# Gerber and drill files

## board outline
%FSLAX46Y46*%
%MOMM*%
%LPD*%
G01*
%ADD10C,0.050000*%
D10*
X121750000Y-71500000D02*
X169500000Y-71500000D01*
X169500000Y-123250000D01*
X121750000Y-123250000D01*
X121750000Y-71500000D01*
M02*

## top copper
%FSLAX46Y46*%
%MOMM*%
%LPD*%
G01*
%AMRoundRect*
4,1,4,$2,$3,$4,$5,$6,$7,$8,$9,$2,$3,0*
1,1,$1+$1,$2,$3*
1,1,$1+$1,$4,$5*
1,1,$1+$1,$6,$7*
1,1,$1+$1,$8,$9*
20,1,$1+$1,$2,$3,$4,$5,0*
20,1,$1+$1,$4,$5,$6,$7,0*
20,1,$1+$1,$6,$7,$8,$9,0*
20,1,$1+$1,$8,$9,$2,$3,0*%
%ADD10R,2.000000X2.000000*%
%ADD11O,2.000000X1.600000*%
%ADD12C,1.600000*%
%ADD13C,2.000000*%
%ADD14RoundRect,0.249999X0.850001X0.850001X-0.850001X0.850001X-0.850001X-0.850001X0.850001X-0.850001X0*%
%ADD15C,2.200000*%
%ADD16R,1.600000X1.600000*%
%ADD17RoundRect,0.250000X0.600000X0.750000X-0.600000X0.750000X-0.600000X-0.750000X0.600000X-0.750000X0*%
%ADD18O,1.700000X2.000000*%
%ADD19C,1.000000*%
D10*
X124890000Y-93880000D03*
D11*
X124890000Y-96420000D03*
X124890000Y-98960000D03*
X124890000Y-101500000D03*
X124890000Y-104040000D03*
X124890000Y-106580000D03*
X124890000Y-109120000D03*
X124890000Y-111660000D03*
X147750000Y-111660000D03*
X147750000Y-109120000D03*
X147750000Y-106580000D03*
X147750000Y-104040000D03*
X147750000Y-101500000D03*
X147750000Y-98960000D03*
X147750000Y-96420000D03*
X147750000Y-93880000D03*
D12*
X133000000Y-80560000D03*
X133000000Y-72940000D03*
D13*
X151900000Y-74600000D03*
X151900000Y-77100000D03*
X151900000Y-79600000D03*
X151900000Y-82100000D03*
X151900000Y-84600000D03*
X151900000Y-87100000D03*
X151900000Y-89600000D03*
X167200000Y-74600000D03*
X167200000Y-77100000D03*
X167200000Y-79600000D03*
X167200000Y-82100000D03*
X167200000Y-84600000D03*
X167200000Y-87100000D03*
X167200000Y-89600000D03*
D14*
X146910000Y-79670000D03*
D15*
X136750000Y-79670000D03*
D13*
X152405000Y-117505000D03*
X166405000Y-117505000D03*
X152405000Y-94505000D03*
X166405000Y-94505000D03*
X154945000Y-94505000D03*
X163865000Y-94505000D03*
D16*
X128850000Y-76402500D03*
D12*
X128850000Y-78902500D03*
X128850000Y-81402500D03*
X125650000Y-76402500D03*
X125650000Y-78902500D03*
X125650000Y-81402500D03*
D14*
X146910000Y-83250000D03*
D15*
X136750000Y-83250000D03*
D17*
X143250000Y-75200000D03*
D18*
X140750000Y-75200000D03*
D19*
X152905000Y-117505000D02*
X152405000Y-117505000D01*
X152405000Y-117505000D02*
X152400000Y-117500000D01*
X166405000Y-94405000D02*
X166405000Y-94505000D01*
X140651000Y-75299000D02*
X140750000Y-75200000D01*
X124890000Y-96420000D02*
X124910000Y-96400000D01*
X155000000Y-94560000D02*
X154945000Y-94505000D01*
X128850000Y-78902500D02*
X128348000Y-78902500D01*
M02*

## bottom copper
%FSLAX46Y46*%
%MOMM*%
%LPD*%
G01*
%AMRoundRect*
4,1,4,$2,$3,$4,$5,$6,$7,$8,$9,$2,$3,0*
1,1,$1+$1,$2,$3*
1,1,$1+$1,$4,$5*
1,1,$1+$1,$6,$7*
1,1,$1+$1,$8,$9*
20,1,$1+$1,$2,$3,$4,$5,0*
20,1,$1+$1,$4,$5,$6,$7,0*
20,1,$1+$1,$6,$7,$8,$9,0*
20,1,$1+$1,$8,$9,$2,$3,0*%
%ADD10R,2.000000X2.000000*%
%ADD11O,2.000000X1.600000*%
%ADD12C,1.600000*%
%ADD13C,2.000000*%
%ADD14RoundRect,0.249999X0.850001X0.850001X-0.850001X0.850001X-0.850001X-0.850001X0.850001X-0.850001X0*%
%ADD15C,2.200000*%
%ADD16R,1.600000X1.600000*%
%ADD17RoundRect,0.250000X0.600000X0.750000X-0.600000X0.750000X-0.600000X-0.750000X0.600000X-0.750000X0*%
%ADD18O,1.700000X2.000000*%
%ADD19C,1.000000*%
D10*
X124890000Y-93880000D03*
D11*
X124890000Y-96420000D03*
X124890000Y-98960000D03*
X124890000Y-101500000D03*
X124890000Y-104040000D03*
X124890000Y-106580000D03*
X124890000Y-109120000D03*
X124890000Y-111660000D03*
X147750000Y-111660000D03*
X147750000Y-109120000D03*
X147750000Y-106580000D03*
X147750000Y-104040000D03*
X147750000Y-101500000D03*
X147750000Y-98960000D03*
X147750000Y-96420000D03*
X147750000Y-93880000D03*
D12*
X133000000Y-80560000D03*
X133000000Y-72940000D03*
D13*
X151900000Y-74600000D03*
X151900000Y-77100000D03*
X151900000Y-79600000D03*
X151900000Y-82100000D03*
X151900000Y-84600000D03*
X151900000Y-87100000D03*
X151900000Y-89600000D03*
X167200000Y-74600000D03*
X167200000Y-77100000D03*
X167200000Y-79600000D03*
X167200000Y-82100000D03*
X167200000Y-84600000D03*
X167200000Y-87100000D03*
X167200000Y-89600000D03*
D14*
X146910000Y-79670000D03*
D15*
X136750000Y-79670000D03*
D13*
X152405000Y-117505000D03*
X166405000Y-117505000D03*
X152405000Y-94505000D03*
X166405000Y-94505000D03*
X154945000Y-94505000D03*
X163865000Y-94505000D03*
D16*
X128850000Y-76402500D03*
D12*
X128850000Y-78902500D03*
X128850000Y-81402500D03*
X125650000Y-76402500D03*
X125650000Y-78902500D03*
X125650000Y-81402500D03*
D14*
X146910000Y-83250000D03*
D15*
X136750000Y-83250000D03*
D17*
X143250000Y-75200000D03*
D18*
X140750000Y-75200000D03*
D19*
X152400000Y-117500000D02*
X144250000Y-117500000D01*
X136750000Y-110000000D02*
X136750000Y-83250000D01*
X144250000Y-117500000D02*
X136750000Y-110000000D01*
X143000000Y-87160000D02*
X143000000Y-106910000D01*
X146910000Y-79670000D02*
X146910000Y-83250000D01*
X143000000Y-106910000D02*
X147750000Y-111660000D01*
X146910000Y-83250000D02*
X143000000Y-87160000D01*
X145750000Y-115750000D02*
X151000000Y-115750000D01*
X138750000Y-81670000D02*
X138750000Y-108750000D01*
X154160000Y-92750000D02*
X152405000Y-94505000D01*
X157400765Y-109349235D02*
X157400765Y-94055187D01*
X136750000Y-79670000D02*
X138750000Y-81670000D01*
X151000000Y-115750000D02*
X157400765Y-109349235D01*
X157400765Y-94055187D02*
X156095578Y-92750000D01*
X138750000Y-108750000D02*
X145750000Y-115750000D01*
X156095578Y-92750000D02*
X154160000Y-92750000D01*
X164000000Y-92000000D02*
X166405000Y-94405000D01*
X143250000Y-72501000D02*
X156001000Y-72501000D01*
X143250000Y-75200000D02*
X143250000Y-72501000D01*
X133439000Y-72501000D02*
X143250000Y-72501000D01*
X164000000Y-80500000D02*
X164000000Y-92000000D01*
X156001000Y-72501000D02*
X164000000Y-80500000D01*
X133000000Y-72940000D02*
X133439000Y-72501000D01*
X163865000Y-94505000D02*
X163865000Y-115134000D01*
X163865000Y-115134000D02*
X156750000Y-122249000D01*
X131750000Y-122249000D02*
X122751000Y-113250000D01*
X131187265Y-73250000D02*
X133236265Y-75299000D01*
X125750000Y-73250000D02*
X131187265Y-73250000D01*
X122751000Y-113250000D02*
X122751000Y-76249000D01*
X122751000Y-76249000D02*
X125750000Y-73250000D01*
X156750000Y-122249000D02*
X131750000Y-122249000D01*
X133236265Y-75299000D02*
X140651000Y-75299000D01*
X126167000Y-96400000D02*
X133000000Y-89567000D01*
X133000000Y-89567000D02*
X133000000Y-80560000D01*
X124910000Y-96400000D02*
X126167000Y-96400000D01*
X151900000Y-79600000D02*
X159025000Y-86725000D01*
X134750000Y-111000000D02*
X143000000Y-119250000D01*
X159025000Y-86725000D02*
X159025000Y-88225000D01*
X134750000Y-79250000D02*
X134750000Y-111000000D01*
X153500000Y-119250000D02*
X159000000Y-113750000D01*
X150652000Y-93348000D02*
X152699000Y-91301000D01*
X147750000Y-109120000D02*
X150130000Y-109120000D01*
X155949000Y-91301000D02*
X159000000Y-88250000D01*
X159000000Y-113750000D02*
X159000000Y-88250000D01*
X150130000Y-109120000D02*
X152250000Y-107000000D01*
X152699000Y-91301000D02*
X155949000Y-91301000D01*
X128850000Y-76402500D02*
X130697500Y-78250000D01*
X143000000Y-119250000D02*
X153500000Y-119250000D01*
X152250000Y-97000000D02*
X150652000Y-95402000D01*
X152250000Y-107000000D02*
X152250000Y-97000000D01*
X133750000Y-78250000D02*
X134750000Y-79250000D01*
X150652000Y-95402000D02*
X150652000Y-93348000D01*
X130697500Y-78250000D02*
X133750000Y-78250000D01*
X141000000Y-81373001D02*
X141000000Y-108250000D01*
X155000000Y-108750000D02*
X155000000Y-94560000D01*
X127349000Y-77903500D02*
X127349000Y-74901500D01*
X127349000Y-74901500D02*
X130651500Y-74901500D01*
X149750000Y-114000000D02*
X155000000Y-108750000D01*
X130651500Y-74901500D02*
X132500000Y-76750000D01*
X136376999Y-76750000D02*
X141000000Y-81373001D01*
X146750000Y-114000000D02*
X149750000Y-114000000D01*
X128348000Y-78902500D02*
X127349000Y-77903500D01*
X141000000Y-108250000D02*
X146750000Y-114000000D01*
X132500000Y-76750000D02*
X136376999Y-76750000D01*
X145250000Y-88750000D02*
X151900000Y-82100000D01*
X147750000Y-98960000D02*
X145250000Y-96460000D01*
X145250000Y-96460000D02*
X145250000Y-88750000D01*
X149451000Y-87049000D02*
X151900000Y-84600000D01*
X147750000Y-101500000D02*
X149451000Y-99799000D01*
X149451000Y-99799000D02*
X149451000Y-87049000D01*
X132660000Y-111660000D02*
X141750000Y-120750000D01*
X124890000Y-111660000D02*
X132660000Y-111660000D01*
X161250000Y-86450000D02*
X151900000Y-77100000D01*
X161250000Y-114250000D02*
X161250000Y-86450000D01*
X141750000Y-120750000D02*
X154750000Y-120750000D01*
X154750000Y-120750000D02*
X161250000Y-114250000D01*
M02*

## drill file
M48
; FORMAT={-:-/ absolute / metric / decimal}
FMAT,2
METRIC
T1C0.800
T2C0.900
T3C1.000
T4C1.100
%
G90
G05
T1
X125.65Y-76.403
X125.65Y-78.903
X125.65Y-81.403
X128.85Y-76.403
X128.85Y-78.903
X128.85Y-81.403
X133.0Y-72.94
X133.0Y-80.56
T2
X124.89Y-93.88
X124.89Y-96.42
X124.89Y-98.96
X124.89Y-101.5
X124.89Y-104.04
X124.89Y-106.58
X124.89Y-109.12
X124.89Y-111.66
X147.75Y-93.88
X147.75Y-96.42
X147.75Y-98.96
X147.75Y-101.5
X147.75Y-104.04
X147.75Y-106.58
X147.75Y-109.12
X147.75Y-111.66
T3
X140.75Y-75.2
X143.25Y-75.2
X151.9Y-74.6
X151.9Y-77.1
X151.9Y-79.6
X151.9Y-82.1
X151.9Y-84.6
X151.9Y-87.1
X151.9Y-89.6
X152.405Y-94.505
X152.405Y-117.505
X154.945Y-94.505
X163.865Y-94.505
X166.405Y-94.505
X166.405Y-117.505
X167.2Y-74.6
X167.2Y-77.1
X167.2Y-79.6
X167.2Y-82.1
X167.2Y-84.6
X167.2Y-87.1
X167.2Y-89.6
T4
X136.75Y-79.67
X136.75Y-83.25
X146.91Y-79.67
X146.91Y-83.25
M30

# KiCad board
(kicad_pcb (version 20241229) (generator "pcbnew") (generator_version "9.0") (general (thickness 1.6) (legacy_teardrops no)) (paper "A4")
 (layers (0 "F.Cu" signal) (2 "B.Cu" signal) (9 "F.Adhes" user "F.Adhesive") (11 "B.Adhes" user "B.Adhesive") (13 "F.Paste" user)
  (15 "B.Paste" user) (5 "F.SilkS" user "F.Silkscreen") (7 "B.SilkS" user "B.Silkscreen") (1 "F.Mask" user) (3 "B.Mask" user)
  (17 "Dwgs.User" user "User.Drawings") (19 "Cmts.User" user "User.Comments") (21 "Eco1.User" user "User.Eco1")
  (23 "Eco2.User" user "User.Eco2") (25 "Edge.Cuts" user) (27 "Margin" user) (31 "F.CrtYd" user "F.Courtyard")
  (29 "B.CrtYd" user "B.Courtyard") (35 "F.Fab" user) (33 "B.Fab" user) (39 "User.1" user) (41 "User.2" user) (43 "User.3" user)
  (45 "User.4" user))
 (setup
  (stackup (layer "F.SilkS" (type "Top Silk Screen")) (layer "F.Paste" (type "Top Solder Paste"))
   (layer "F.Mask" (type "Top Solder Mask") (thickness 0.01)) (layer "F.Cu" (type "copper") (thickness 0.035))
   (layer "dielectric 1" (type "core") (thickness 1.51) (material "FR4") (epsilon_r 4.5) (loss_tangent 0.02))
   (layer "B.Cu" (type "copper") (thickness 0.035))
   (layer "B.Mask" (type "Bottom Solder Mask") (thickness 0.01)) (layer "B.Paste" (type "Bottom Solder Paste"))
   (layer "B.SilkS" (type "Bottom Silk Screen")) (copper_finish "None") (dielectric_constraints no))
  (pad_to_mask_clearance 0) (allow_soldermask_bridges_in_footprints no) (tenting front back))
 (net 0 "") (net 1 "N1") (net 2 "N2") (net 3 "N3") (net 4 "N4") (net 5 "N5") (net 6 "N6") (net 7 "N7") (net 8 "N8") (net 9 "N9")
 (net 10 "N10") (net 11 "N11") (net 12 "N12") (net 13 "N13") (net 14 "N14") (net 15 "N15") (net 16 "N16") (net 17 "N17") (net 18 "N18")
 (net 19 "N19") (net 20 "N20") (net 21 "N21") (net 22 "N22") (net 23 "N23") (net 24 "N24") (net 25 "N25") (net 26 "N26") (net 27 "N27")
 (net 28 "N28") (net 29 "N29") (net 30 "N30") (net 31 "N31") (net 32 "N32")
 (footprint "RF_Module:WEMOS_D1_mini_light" (layer "F.Cu") (at 124.89 93.88)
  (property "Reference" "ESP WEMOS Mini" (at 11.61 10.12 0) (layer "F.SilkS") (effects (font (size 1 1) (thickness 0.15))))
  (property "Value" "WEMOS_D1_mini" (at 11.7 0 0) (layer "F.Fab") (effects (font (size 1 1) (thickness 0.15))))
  (pad "1" thru_hole rect (at 0 0) (size 2 2) (drill 0.9) (layers "*.Cu" "*.Mask") (remove_unused_layers no) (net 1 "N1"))
  (pad "2" thru_hole oval (at 0 2.54) (size 2 1.6) (drill 0.9) (layers "*.Cu" "*.Mask") (remove_unused_layers no) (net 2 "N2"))
  (pad "3" thru_hole oval (at 0 5.08) (size 2 1.6) (drill 0.9) (layers "*.Cu" "*.Mask") (remove_unused_layers no) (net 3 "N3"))
  (pad "4" thru_hole oval (at 0 7.62) (size 2 1.6) (drill 0.9) (layers "*.Cu" "*.Mask") (remove_unused_layers no) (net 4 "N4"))
  (pad "5" thru_hole oval (at 0 10.16) (size 2 1.6) (drill 0.9) (layers "*.Cu" "*.Mask") (remove_unused_layers no) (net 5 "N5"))
  (pad "6" thru_hole oval (at 0 12.7) (size 2 1.6) (drill 0.9) (layers "*.Cu" "*.Mask") (remove_unused_layers no) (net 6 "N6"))
  (pad "7" thru_hole oval (at 0 15.24) (size 2 1.6) (drill 0.9) (layers "*.Cu" "*.Mask") (remove_unused_layers no) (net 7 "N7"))
  (pad "8" thru_hole oval (at 0 17.78) (size 2 1.6) (drill 0.9) (layers "*.Cu" "*.Mask") (remove_unused_layers no) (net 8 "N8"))
  (pad "9" thru_hole oval (at 22.86 17.78) (size 2 1.6) (drill 0.9) (layers "*.Cu" "*.Mask") (remove_unused_layers no) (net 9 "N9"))
  (pad "10" thru_hole oval (at 22.86 15.24) (size 2 1.6) (drill 0.9) (layers "*.Cu" "*.Mask") (remove_unused_layers no) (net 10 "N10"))
  (pad "11" thru_hole oval (at 22.86 12.7) (size 2 1.6) (drill 0.9) (layers "*.Cu" "*.Mask") (remove_unused_layers no) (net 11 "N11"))
  (pad "12" thru_hole oval (at 22.86 10.16) (size 2 1.6) (drill 0.9) (layers "*.Cu" "*.Mask") (remove_unused_layers no) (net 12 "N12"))
  (pad "13" thru_hole oval (at 22.86 7.62) (size 2 1.6) (drill 0.9) (layers "*.Cu" "*.Mask") (remove_unused_layers no) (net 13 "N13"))
  (pad "14" thru_hole oval (at 22.86 5.08) (size 2 1.6) (drill 0.9) (layers "*.Cu" "*.Mask") (remove_unused_layers no) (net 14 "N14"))
  (pad "15" thru_hole oval (at 22.86 2.54) (size 2 1.6) (drill 0.9) (layers "*.Cu" "*.Mask") (remove_unused_layers no) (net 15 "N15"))
  (pad "16" thru_hole oval (at 22.86 0) (size 2 1.6) (drill 0.9) (layers "*.Cu" "*.Mask") (remove_unused_layers no) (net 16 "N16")))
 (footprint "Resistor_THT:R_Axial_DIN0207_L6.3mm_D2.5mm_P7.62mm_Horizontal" (layer "F.Cu") (at 133 80.56 90)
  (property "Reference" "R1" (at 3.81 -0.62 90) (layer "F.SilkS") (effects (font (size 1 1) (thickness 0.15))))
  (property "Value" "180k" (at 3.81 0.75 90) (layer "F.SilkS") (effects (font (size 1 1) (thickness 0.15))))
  (pad "1" thru_hole circle (at 0 0 90) (size 1.6 1.6) (drill 0.8) (layers "*.Cu" "*.Mask") (remove_unused_layers no) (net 2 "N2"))
  (pad "2" thru_hole circle (at 7.62 0 90) (size 1.6 1.6) (drill 0.8) (layers "*.Cu" "*.Mask") (remove_unused_layers no) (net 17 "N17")))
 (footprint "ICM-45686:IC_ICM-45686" (layer "F.Cu") (at 160.5 82)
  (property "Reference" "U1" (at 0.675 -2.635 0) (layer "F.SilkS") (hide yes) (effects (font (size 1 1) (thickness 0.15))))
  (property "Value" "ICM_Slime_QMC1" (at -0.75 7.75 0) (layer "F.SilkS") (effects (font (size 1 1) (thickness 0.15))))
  (pad "1" thru_hole circle (at -8.6 -7.4) (size 2 2) (drill 1) (layers "*.Cu" "*.Mask") (remove_unused_layers no) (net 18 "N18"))
  (pad "2" thru_hole circle (at -8.6 -4.9) (size 2 2) (drill 1) (layers "*.Cu" "*.Mask") (remove_unused_layers no) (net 8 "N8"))
  (pad "3" thru_hole circle (at -8.6 -2.4) (size 2 2) (drill 1) (layers "*.Cu" "*.Mask") (remove_unused_layers no) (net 10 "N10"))
  (pad "4" thru_hole circle (at -8.6 0.1) (size 2 2) (drill 1) (layers "*.Cu" "*.Mask") (remove_unused_layers no) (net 14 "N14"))
  (pad "5" thru_hole circle (at -8.6 2.6) (size 2 2) (drill 1) (layers "*.Cu" "*.Mask") (remove_unused_layers no) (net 13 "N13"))
  (pad "6" thru_hole circle (at -8.6 5.1) (size 2 2) (drill 1) (layers "*.Cu" "*.Mask") (remove_unused_layers no) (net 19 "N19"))
  (pad "7" thru_hole circle (at -8.6 7.6) (size 2 2) (drill 1) (layers "*.Cu" "*.Mask") (remove_unused_layers no) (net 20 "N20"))
  (pad "8" thru_hole circle (at 6.7 -7.4) (size 2 2) (drill 1) (layers "*.Cu" "*.Mask") (remove_unused_layers no) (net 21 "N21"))
  (pad "9" thru_hole circle (at 6.7 -4.9) (size 2 2) (drill 1) (layers "*.Cu" "*.Mask") (remove_unused_layers no) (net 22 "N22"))
  (pad "10" thru_hole circle (at 6.7 -2.4) (size 2 2) (drill 1) (layers "*.Cu" "*.Mask") (remove_unused_layers no) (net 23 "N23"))
  (pad "11" thru_hole circle (at 6.7 0.1) (size 2 2) (drill 1) (layers "*.Cu" "*.Mask") (remove_unused_layers no) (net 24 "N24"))
  (pad "12" thru_hole circle (at 6.7 2.6) (size 2 2) (drill 1) (layers "*.Cu" "*.Mask") (remove_unused_layers no) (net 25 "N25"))
  (pad "13" thru_hole circle (at 6.7 5.1) (size 2 2) (drill 1) (layers "*.Cu" "*.Mask") (remove_unused_layers no) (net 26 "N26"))
  (pad "14" thru_hole circle (at 6.7 7.6) (size 2 2) (drill 1) (layers "*.Cu" "*.Mask") (remove_unused_layers no) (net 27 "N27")))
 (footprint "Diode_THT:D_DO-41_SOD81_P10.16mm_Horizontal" (layer "F.Cu") (at 146.91 79.67 180)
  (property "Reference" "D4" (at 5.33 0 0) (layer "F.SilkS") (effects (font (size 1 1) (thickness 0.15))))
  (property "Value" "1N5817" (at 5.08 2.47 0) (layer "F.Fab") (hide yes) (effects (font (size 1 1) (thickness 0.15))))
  (pad "1" thru_hole roundrect (at 0 0 180) (size 2.2 2.2) (drill 1.1) (layers "*.Cu" "*.Mask") (remove_unused_layers no)
   (roundrect_rratio 0.113636) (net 9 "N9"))
  (pad "2" thru_hole circle (at 10.16 0 180) (size 2.2 2.2) (drill 1.1) (layers "*.Cu" "*.Mask") (remove_unused_layers no) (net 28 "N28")))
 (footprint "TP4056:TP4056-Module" (layer "F.Cu") (at 168.005 120.005 90)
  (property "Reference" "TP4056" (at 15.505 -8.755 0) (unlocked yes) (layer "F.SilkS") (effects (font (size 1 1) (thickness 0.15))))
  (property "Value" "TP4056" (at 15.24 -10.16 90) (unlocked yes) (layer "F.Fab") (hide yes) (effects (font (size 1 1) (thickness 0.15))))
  (pad "1" thru_hole circle (at 2.5 -15.6 90) (size 2 2) (drill 1) (layers "*.Cu" "*.Mask") (remove_unused_layers no) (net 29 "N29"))
  (pad "2" thru_hole circle (at 2.5 -1.6 90) (size 2 2) (drill 1) (layers "*.Cu" "*.Mask") (remove_unused_layers no) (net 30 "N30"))
  (pad "3" thru_hole circle (at 25.5 -15.6 90) (size 2 2) (drill 1) (layers "*.Cu" "*.Mask") (remove_unused_layers no) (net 28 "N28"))
  (pad "4" thru_hole circle (at 25.5 -1.6 90) (size 2 2) (drill 1) (layers "*.Cu" "*.Mask") (remove_unused_layers no) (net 17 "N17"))
  (pad "5" thru_hole circle (at 25.5 -13.06 90) (size 2 2) (drill 1) (layers "*.Cu" "*.Mask") (remove_unused_layers no) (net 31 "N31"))
  (pad "6" thru_hole circle (at 25.5 -4.14 90) (size 2 2) (drill 1) (layers "*.Cu" "*.Mask") (remove_unused_layers no) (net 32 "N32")))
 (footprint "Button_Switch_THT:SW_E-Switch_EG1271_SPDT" (layer "F.Cu") (at 128.85 76.4025 -90)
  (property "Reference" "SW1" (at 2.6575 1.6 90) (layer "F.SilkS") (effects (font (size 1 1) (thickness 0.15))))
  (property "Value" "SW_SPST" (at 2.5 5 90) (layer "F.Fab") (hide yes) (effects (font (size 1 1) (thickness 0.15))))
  (pad "1" thru_hole rect (at 0 0 270) (size 1.6 1.6) (drill 0.8) (layers "*.Cu" "*.Mask") (remove_unused_layers no) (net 10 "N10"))
  (pad "2" thru_hole circle (at 2.5 0 270) (size 1.6 1.6) (drill 0.8) (layers "*.Cu" "*.Mask") (remove_unused_layers no) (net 31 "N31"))
  (pad "3" thru_hole circle (at 5 0 270) (size 1.6 1.6) (drill 0.8) (layers "*.Cu" "*.Mask") (remove_unused_layers no))
  (pad "4" thru_hole circle (at 0 3.2 270) (size 1.6 1.6) (drill 0.8) (layers "*.Cu" "*.Mask") (remove_unused_layers no))
  (pad "5" thru_hole circle (at 2.5 3.2 270) (size 1.6 1.6) (drill 0.8) (layers "*.Cu" "*.Mask") (remove_unused_layers no))
  (pad "6" thru_hole circle (at 5 3.2 270) (size 1.6 1.6) (drill 0.8) (layers "*.Cu" "*.Mask") (remove_unused_layers no)))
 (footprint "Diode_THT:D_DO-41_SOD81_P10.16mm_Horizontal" (layer "F.Cu") (at 146.91 83.25 180)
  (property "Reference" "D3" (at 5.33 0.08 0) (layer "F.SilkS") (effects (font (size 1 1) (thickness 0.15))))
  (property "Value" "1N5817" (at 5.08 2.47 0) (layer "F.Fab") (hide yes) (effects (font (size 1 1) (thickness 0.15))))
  (pad "1" thru_hole roundrect (at 0 0 180) (size 2.2 2.2) (drill 1.1) (layers "*.Cu" "*.Mask") (remove_unused_layers no)
   (roundrect_rratio 0.113636) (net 9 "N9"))
  (pad "2" thru_hole circle (at 10.16 0 180) (size 2.2 2.2) (drill 1.1) (layers "*.Cu" "*.Mask") (remove_unused_layers no) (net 29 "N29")))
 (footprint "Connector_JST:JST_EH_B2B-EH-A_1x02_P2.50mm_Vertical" (layer "B.Cu") (at 143.25 75.2 180)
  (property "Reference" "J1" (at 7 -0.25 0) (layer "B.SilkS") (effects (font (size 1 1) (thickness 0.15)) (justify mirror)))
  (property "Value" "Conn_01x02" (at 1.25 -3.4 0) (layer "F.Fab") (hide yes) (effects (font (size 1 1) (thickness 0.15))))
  (pad "1" thru_hole roundrect (at 0 0 180) (size 1.7 2) (drill 1) (layers "*.Cu" "*.Mask") (remove_unused_layers no)
   (roundrect_rratio 0.147059) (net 17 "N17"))
  (pad "2" thru_hole oval (at 2.5 0 180) (size 1.7 2) (drill 1) (layers "*.Cu" "*.Mask") (remove_unused_layers no) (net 32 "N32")))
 (gr_rect (start 121.75 71.5) (end 169.5 123.25) (stroke (width 0.05) (type default)) (fill no) (locked yes) (layer "Edge.Cuts"))
 (segment (start 152.905 117.505) (end 152.405 117.505) (width 1) (layer "F.Cu") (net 29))
 (segment (start 152.405 117.505) (end 152.4 117.5) (width 1) (layer "F.Cu") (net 29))
 (segment (start 152.4 117.5) (end 144.25 117.5) (width 1) (layer "B.Cu") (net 29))
 (segment (start 136.75 110) (end 136.75 83.25) (width 1) (layer "B.Cu") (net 29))
 (segment (start 144.25 117.5) (end 136.75 110) (width 1) (layer "B.Cu") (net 29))
 (segment (start 143 87.16) (end 143 106.91) (width 1) (layer "B.Cu") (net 9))
 (segment (start 146.91 79.67) (end 146.91 83.25) (width 1) (layer "B.Cu") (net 9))
 (segment (start 143 106.91) (end 147.75 111.66) (width 1) (layer "B.Cu") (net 9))
 (segment (start 146.91 83.25) (end 143 87.16) (width 1) (layer "B.Cu") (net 9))
 (segment (start 145.75 115.75) (end 151 115.75) (width 1) (layer "B.Cu") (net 28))
 (segment (start 138.75 81.67) (end 138.75 108.75) (width 1) (layer "B.Cu") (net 28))
 (segment (start 154.16 92.75) (end 152.405 94.505) (width 1) (layer "B.Cu") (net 28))
 (segment (start 157.400765 109.349235) (end 157.400765 94.055187) (width 1) (layer "B.Cu") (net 28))
 (segment (start 136.75 79.67) (end 138.75 81.67) (width 1) (layer "B.Cu") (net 28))
 (segment (start 151 115.75) (end 157.400765 109.349235) (width 1) (layer "B.Cu") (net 28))
 (segment (start 157.400765 94.055187) (end 156.095578 92.75) (width 1) (layer "B.Cu") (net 28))
 (segment (start 138.75 108.75) (end 145.75 115.75) (width 1) (layer "B.Cu") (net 28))
 (segment (start 156.095578 92.75) (end 154.16 92.75) (width 1) (layer "B.Cu") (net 28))
 (segment (start 166.405 94.405) (end 166.405 94.505) (width 1) (layer "F.Cu") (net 17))
 (segment (start 164 92) (end 166.405 94.405) (width 1) (layer "B.Cu") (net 17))
 (segment (start 143.25 72.501) (end 156.001 72.501) (width 1) (layer "B.Cu") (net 17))
 (segment (start 143.25 75.2) (end 143.25 72.501) (width 1) (layer "B.Cu") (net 17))
 (segment (start 133.439 72.501) (end 143.25 72.501) (width 1) (layer "B.Cu") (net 17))
 (segment (start 164 80.5) (end 164 92) (width 1) (layer "B.Cu") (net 17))
 (segment (start 156.001 72.501) (end 164 80.5) (width 1) (layer "B.Cu") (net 17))
 (segment (start 133 72.94) (end 133.439 72.501) (width 1) (layer "B.Cu") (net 17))
 (segment (start 140.651 75.299) (end 140.75 75.2) (width 1) (layer "F.Cu") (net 32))
 (segment (start 163.865 94.505) (end 163.865 115.134) (width 1) (layer "B.Cu") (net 32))
 (segment (start 163.865 115.134) (end 156.75 122.249) (width 1) (layer "B.Cu") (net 32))
 (segment (start 131.75 122.249) (end 122.751 113.25) (width 1) (layer "B.Cu") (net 32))
 (segment (start 131.187265 73.25) (end 133.236265 75.299) (width 1) (layer "B.Cu") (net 32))
 (segment (start 125.75 73.25) (end 131.187265 73.25) (width 1) (layer "B.Cu") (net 32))
 (segment (start 122.751 113.25) (end 122.751 76.249) (width 1) (layer "B.Cu") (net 32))
 (segment (start 122.751 76.249) (end 125.75 73.25) (width 1) (layer "B.Cu") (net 32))
 (segment (start 156.75 122.249) (end 131.75 122.249) (width 1) (layer "B.Cu") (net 32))
 (segment (start 133.236265 75.299) (end 140.651 75.299) (width 1) (layer "B.Cu") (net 32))
 (segment (start 124.89 96.42) (end 124.91 96.4) (width 1) (layer "F.Cu") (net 2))
 (segment (start 126.167 96.4) (end 133 89.567) (width 1) (layer "B.Cu") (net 2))
 (segment (start 133 89.567) (end 133 80.56) (width 1) (layer "B.Cu") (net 2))
 (segment (start 124.91 96.4) (end 126.167 96.4) (width 1) (layer "B.Cu") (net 2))
 (segment (start 151.9 79.6) (end 159.025 86.725) (width 1) (layer "B.Cu") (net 10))
 (segment (start 134.75 111) (end 143 119.25) (width 1) (layer "B.Cu") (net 10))
 (segment (start 159.025 86.725) (end 159.025 88.225) (width 1) (layer "B.Cu") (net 10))
 (segment (start 134.75 79.25) (end 134.75 111) (width 1) (layer "B.Cu") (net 10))
 (segment (start 153.5 119.25) (end 159 113.75) (width 1) (layer "B.Cu") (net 10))
 (segment (start 150.652 93.348) (end 152.699 91.301) (width 1) (layer "B.Cu") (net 10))
 (segment (start 147.75 109.12) (end 150.13 109.12) (width 1) (layer "B.Cu") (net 10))
 (segment (start 155.949 91.301) (end 159 88.25) (width 1) (layer "B.Cu") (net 10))
 (segment (start 159 113.75) (end 159 88.25) (width 1) (layer "B.Cu") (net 10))
 (segment (start 150.13 109.12) (end 152.25 107) (width 1) (layer "B.Cu") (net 10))
 (segment (start 152.699 91.301) (end 155.949 91.301) (width 1) (layer "B.Cu") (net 10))
 (segment (start 128.85 76.4025) (end 130.6975 78.25) (width 1) (layer "B.Cu") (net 10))
 (segment (start 143 119.25) (end 153.5 119.25) (width 1) (layer "B.Cu") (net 10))
 (segment (start 152.25 97) (end 150.652 95.402) (width 1) (layer "B.Cu") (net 10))
 (segment (start 152.25 107) (end 152.25 97) (width 1) (layer "B.Cu") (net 10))
 (segment (start 133.75 78.25) (end 134.75 79.25) (width 1) (layer "B.Cu") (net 10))
 (segment (start 150.652 95.402) (end 150.652 93.348) (width 1) (layer "B.Cu") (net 10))
 (segment (start 130.6975 78.25) (end 133.75 78.25) (width 1) (layer "B.Cu") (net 10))
 (segment (start 155 94.56) (end 154.945 94.505) (width 1) (layer "F.Cu") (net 31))
 (segment (start 128.85 78.9025) (end 128.348 78.9025) (width 1) (layer "F.Cu") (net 31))
 (segment (start 141 81.373001) (end 141 108.25) (width 1) (layer "B.Cu") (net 31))
 (segment (start 155 108.75) (end 155 94.56) (width 1) (layer "B.Cu") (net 31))
 (segment (start 127.349 77.9035) (end 127.349 74.9015) (width 1) (layer "B.Cu") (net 31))
 (segment (start 127.349 74.9015) (end 130.6515 74.9015) (width 1) (layer "B.Cu") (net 31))
 (segment (start 149.75 114) (end 155 108.75) (width 1) (layer "B.Cu") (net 31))
 (segment (start 130.6515 74.9015) (end 132.5 76.75) (width 1) (layer "B.Cu") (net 31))
 (segment (start 136.376999 76.75) (end 141 81.373001) (width 1) (layer "B.Cu") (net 31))
 (segment (start 146.75 114) (end 149.75 114) (width 1) (layer "B.Cu") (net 31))
 (segment (start 128.348 78.9025) (end 127.349 77.9035) (width 1) (layer "B.Cu") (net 31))
 (segment (start 141 108.25) (end 146.75 114) (width 1) (layer "B.Cu") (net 31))
 (segment (start 132.5 76.75) (end 136.376999 76.75) (width 1) (layer "B.Cu") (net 31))
 (segment (start 145.25 88.75) (end 151.9 82.1) (width 1) (layer "B.Cu") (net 14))
 (segment (start 147.75 98.96) (end 145.25 96.46) (width 1) (layer "B.Cu") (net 14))
 (segment (start 145.25 96.46) (end 145.25 88.75) (width 1) (layer "B.Cu") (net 14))
 (segment (start 149.451 87.049) (end 151.9 84.6) (width 1) (layer "B.Cu") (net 13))
 (segment (start 147.75 101.5) (end 149.451 99.799) (width 1) (layer "B.Cu") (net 13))
 (segment (start 149.451 99.799) (end 149.451 87.049) (width 1) (layer "B.Cu") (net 13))
 (segment (start 132.66 111.66) (end 141.75 120.75) (width 1) (layer "B.Cu") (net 8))
 (segment (start 124.89 111.66) (end 132.66 111.66) (width 1) (layer "B.Cu") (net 8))
 (segment (start 161.25 86.45) (end 151.9 77.1) (width 1) (layer "B.Cu") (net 8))
 (segment (start 161.25 114.25) (end 161.25 86.45) (width 1) (layer "B.Cu") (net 8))
 (segment (start 141.75 120.75) (end 154.75 120.75) (width 1) (layer "B.Cu") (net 8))
 (segment (start 154.75 120.75) (end 161.25 114.25) (width 1) (layer "B.Cu") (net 8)))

